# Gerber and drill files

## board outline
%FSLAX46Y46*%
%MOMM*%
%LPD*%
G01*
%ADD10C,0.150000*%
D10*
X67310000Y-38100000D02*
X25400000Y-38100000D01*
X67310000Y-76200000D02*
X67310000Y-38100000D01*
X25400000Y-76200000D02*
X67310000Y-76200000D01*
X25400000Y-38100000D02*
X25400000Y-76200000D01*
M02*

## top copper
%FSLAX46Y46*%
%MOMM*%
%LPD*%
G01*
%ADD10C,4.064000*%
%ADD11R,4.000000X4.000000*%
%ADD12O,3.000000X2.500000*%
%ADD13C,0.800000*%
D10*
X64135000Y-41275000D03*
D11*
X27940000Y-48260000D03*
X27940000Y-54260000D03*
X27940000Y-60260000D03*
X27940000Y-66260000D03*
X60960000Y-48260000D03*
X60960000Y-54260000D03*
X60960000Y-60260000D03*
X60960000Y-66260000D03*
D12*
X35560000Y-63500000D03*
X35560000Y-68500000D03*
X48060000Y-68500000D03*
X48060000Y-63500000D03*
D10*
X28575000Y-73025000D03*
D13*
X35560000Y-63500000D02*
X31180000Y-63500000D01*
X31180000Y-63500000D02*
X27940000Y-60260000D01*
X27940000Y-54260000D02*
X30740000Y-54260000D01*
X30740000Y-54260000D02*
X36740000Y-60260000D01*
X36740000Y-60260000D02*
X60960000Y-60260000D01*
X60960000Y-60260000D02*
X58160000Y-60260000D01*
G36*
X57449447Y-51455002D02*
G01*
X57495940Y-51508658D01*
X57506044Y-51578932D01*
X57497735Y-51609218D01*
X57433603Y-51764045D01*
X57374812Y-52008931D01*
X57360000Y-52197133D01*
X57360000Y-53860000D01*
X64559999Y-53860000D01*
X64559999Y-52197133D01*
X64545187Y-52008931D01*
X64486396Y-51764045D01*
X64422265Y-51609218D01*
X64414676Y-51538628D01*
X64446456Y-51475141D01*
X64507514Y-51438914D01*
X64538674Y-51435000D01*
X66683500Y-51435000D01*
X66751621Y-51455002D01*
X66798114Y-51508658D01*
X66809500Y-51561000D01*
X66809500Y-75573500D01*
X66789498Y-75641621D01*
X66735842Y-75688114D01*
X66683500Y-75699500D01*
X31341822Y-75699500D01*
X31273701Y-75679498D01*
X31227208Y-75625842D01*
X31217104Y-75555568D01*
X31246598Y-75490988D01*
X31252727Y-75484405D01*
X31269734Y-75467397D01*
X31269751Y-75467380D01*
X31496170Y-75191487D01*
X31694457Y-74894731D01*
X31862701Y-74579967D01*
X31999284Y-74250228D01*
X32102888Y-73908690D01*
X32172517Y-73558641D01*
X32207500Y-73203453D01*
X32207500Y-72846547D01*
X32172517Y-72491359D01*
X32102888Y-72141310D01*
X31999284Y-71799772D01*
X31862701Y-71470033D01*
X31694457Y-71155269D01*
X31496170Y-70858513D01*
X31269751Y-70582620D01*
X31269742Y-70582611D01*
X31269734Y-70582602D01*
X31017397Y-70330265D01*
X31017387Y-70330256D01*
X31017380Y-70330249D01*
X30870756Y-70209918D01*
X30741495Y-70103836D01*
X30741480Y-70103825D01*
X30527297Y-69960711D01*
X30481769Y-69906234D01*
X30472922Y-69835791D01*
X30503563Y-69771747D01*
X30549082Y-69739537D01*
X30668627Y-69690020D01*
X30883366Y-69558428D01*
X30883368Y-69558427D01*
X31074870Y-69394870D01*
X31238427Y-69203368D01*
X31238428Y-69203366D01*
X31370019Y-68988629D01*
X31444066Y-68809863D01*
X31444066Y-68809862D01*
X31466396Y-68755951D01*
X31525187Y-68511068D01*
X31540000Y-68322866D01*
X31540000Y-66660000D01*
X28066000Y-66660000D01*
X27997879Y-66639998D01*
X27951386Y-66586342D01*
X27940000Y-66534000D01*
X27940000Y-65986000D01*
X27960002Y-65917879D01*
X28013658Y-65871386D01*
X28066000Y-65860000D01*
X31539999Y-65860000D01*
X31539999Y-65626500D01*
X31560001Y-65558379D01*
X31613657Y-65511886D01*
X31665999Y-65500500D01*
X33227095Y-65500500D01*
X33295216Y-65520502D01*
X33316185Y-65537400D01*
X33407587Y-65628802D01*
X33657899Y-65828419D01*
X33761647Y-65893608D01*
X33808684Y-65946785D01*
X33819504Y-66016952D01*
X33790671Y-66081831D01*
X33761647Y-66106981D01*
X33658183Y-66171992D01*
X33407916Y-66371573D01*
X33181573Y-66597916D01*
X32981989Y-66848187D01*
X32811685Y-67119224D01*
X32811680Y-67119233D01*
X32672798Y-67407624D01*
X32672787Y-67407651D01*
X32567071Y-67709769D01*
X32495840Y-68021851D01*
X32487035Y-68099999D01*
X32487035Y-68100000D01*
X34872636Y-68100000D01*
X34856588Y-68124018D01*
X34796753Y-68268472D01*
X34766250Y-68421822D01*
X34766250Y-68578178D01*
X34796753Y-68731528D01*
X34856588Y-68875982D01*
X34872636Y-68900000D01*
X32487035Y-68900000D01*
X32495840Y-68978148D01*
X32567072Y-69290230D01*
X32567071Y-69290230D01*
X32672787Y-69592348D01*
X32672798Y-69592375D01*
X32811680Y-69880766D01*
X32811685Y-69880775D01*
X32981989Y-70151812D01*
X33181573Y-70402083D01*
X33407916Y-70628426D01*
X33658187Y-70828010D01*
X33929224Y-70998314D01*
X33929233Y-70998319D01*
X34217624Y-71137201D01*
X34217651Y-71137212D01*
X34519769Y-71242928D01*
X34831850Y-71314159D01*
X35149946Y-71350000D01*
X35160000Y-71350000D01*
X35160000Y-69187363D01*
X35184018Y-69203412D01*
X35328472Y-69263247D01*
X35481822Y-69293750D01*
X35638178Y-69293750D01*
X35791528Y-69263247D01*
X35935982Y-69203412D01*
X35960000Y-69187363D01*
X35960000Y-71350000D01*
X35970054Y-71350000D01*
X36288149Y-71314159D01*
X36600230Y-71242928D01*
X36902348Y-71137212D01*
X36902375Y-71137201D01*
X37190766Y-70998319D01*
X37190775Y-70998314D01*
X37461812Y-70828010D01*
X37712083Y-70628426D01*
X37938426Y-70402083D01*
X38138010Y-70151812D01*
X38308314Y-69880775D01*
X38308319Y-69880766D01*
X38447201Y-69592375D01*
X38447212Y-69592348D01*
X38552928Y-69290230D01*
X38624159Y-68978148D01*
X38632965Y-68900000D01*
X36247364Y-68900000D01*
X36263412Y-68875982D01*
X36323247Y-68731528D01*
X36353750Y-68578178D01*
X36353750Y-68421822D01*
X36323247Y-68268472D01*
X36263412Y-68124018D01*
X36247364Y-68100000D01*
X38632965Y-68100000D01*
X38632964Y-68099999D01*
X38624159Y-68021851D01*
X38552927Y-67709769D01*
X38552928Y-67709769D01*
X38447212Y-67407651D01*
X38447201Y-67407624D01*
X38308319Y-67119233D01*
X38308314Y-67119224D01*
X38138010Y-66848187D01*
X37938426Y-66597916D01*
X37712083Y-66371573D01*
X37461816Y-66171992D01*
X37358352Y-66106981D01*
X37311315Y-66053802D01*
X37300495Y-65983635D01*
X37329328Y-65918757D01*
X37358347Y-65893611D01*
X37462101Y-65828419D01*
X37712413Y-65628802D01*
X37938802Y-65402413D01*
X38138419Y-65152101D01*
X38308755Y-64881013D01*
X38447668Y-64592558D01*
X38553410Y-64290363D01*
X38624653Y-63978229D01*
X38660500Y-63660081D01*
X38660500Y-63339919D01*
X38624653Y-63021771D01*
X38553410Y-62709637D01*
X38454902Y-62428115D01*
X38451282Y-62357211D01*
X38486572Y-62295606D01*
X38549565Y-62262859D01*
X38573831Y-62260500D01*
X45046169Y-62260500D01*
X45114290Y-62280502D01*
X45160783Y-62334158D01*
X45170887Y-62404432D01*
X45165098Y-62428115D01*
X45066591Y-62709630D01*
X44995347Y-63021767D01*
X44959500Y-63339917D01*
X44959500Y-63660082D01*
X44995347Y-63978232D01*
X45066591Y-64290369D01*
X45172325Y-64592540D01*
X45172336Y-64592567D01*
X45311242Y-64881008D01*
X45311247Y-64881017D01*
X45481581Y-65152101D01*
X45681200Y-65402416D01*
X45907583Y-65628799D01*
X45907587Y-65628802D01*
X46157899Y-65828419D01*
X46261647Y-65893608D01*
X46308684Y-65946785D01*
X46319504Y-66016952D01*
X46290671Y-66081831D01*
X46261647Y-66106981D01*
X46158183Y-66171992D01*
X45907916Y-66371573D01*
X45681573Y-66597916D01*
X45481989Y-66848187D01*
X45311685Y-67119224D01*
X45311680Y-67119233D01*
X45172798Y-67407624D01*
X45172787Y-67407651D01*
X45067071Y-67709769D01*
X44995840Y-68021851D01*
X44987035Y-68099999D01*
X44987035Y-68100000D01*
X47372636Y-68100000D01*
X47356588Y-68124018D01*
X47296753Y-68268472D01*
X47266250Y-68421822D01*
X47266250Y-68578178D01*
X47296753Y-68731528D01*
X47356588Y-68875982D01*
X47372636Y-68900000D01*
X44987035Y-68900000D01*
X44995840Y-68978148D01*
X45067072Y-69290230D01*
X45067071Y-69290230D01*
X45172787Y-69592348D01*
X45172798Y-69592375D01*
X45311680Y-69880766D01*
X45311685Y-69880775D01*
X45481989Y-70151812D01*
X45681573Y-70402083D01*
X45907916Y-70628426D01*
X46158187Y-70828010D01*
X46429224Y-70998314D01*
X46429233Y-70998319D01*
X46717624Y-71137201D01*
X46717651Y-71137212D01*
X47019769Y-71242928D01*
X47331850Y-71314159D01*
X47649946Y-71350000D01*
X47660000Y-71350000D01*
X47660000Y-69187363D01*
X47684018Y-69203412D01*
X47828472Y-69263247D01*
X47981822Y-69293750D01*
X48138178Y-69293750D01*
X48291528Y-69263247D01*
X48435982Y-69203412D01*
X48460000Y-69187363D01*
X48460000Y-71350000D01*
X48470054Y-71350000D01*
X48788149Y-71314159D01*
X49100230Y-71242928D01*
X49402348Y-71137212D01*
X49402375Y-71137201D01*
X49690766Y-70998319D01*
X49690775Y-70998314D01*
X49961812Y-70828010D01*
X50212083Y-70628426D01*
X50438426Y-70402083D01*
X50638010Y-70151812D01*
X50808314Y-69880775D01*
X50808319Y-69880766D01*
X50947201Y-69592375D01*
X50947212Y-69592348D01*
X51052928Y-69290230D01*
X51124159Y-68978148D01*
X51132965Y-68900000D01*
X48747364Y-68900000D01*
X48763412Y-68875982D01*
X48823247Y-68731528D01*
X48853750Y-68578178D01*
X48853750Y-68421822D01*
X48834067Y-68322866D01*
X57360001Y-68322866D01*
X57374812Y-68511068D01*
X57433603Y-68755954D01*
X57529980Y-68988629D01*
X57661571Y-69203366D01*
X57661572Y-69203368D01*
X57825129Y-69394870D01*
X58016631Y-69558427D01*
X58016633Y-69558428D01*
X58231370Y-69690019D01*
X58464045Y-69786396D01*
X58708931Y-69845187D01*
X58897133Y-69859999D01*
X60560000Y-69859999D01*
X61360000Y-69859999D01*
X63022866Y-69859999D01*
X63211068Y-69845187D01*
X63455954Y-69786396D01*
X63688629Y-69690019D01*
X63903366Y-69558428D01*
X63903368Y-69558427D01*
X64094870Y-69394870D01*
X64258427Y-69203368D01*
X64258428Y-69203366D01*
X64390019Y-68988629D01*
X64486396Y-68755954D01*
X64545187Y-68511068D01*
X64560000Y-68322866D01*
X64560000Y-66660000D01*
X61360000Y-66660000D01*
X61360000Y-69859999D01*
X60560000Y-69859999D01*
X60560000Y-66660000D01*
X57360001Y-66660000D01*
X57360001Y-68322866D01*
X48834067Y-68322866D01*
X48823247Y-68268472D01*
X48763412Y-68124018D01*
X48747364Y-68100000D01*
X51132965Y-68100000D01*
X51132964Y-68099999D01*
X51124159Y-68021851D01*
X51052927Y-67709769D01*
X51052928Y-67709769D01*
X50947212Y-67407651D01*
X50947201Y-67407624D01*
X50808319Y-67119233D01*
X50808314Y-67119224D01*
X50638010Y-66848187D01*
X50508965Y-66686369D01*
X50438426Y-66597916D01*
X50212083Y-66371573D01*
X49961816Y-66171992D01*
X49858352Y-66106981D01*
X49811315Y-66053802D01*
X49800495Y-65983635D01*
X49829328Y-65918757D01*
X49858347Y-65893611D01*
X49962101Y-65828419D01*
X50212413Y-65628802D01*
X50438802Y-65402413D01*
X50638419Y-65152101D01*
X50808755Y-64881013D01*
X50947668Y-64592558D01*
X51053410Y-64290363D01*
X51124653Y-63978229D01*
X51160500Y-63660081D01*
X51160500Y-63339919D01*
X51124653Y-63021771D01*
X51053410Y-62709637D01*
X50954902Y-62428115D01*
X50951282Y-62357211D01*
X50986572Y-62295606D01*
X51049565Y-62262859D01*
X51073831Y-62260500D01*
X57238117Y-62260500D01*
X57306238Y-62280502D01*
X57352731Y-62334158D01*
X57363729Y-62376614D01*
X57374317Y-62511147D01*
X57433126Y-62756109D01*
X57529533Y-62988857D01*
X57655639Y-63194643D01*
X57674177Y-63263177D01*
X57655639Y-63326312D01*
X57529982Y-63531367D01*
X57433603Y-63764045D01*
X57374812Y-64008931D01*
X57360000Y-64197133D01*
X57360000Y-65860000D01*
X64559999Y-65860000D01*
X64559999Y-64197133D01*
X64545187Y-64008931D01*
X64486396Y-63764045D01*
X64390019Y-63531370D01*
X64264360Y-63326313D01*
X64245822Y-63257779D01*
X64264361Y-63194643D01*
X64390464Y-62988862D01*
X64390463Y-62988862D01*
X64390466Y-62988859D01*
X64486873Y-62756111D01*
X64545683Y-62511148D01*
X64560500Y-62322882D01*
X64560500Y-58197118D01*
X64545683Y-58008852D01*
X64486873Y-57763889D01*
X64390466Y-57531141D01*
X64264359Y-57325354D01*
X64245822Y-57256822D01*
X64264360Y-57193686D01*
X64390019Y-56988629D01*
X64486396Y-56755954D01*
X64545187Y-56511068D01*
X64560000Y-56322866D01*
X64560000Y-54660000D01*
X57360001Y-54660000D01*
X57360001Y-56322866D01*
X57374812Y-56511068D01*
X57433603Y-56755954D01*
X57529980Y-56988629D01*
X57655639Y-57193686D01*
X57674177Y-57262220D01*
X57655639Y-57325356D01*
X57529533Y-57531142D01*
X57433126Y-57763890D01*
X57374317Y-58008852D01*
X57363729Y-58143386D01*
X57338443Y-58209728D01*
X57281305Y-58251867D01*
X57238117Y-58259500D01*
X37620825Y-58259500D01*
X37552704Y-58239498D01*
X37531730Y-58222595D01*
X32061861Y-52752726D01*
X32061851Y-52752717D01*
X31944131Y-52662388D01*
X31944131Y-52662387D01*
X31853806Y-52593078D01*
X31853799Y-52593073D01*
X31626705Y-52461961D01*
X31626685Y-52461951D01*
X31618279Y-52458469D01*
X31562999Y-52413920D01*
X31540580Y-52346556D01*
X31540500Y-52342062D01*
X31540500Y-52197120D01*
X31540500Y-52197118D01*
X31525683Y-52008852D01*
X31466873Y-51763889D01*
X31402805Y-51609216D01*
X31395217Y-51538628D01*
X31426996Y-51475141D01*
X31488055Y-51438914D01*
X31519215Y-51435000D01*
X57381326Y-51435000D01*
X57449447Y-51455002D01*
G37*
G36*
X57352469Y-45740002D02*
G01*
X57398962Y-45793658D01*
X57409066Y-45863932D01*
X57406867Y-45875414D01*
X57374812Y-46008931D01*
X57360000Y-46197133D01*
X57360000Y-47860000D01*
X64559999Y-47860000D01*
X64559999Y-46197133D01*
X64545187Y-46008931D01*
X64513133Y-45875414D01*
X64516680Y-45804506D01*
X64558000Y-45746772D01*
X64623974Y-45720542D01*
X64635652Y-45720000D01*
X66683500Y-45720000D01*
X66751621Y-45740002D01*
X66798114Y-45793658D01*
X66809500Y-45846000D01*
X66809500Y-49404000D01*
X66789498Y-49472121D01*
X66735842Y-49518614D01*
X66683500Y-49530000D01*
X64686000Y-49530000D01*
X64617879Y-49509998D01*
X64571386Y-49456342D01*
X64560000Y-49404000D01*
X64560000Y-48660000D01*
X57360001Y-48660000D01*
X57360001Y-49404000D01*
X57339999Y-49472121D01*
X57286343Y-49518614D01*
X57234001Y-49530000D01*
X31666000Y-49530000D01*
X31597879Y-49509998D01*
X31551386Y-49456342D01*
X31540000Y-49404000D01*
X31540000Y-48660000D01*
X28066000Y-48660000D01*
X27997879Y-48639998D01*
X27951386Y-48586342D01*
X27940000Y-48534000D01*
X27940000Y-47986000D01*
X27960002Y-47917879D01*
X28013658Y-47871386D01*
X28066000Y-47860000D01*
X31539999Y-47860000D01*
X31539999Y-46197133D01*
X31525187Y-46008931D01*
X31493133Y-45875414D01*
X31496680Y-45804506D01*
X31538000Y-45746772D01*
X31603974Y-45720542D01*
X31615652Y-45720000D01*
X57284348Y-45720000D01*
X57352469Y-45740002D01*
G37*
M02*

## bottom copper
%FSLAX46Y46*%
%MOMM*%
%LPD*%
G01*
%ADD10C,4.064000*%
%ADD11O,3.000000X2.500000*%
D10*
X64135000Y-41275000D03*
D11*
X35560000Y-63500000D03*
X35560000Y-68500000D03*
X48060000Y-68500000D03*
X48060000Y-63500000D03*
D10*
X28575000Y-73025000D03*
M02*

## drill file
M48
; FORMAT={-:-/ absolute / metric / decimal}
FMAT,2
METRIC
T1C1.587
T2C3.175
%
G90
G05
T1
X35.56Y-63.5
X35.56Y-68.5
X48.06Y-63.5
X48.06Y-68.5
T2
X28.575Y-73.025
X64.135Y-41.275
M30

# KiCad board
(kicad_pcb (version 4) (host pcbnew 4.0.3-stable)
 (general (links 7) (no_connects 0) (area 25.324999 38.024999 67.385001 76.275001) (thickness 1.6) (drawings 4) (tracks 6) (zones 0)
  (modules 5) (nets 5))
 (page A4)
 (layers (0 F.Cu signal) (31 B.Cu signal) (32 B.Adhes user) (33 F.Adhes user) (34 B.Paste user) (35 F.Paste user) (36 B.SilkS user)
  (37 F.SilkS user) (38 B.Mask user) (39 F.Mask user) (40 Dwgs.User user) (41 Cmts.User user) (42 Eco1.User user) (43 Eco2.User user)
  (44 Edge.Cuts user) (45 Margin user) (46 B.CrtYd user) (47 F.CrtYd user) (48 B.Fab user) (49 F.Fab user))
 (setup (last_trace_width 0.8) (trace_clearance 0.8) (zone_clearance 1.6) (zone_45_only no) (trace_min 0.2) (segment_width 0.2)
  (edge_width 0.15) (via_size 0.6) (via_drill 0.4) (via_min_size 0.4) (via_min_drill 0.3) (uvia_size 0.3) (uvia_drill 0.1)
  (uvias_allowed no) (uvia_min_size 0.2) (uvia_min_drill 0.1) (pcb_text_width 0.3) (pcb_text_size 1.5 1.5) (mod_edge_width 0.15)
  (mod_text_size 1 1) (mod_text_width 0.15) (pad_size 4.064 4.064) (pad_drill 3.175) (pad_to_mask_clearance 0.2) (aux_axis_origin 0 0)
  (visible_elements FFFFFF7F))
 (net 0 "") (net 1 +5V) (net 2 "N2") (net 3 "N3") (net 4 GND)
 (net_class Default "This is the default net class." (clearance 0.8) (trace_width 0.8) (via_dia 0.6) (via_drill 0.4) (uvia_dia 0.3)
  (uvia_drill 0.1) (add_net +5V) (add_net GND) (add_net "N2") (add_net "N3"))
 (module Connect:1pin (layer F.Cu) (at 64.135 41.275)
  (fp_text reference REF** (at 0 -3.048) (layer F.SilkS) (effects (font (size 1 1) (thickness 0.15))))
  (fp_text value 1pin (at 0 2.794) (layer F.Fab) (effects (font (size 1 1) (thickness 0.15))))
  (pad 1 thru_hole circle (at 0 0) (size 4.064 4.064) (drill 3.175) (layers *.Cu *.Mask F.SilkS)))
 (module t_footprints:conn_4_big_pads (layer F.Cu) (at 27.94 48.26)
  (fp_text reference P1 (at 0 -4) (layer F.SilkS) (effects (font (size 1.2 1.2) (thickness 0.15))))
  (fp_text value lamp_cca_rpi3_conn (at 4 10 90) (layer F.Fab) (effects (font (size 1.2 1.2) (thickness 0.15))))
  (pad 1 smd rect (at 0 0) (size 4 4) (layers F.Cu F.Paste F.Mask) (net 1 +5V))
  (pad 2 smd rect (at 0 6) (size 4 4) (layers F.Cu F.Paste F.Mask) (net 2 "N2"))
  (pad 3 smd rect (at 0 12) (size 4 4) (layers F.Cu F.Paste F.Mask) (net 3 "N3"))
  (pad 4 smd rect (at 0 18) (size 4 4) (layers F.Cu F.Paste F.Mask) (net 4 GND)))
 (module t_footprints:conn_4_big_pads (layer F.Cu) (at 60.96 48.26)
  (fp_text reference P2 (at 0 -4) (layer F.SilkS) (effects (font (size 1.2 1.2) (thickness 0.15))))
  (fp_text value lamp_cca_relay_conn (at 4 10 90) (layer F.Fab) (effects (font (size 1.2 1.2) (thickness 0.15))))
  (pad 1 smd rect (at 0 0) (size 4 4) (layers F.Cu F.Paste F.Mask) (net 1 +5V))
  (pad 2 smd rect (at 0 6) (size 4 4) (layers F.Cu F.Paste F.Mask) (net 4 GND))
  (pad 3 smd rect (at 0 12) (size 4 4) (layers F.Cu F.Paste F.Mask) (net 2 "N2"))
  (pad 4 smd rect (at 0 18) (size 4 4) (layers F.Cu F.Paste F.Mask) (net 4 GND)))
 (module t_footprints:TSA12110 (layer F.Cu) (at 35.56 63.5)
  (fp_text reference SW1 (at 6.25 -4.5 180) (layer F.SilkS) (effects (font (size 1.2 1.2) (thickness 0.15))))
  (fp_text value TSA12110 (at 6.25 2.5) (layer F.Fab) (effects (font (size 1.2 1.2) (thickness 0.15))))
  (pad 1 thru_hole oval (at 0 0) (size 3 2.5) (drill 1.5875) (layers *.Cu *.Mask) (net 3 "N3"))
  (pad 3 thru_hole oval (at 0 5) (size 3 2.5) (drill 1.5875) (layers *.Cu *.Mask) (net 4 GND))
  (pad 4 thru_hole oval (at 12.5 5) (size 3 2.5) (drill 1.5875) (layers *.Cu *.Mask) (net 4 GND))
  (pad 2 thru_hole oval (at 12.5 0) (size 3 2.5) (drill 1.5875) (layers *.Cu *.Mask)))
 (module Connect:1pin (layer F.Cu) (at 28.575 73.025)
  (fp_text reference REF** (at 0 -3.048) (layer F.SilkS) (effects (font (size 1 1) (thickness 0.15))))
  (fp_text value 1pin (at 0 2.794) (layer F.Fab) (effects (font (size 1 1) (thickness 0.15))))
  (pad 1 thru_hole circle (at 0 0) (size 4.064 4.064) (drill 3.175) (layers *.Cu *.Mask F.SilkS)))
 (gr_line (start 67.31 38.1) (end 25.4 38.1) (angle 90) (layer Edge.Cuts) (width 0.15))
 (gr_line (start 67.31 76.2) (end 67.31 38.1) (angle 90) (layer Edge.Cuts) (width 0.15))
 (gr_line (start 25.4 76.2) (end 67.31 76.2) (angle 90) (layer Edge.Cuts) (width 0.15))
 (gr_line (start 25.4 38.1) (end 25.4 76.2) (angle 90) (layer Edge.Cuts) (width 0.15))
 (segment (start 35.56 63.5) (end 31.18 63.5) (width 0.8) (layer F.Cu) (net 3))
 (segment (start 31.18 63.5) (end 27.94 60.26) (width 0.8) (layer F.Cu) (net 3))
 (segment (start 27.94 54.26) (end 30.74 54.26) (width 0.8) (layer F.Cu) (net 2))
 (segment (start 30.74 54.26) (end 36.74 60.26) (width 0.8) (layer F.Cu) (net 2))
 (segment (start 36.74 60.26) (end 60.96 60.26) (width 0.8) (layer F.Cu) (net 2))
 (segment (start 60.96 60.26) (end 58.16 60.26) (width 0.8) (layer F.Cu) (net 2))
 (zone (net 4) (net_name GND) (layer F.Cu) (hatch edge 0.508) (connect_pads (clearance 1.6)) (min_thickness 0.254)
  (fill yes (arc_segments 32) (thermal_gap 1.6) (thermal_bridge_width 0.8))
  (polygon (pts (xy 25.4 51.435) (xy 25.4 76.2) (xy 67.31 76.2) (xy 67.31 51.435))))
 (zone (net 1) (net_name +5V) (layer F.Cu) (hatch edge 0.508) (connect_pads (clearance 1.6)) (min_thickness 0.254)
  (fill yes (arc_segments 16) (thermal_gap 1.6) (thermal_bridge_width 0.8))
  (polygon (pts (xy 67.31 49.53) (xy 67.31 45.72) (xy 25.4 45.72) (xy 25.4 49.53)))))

